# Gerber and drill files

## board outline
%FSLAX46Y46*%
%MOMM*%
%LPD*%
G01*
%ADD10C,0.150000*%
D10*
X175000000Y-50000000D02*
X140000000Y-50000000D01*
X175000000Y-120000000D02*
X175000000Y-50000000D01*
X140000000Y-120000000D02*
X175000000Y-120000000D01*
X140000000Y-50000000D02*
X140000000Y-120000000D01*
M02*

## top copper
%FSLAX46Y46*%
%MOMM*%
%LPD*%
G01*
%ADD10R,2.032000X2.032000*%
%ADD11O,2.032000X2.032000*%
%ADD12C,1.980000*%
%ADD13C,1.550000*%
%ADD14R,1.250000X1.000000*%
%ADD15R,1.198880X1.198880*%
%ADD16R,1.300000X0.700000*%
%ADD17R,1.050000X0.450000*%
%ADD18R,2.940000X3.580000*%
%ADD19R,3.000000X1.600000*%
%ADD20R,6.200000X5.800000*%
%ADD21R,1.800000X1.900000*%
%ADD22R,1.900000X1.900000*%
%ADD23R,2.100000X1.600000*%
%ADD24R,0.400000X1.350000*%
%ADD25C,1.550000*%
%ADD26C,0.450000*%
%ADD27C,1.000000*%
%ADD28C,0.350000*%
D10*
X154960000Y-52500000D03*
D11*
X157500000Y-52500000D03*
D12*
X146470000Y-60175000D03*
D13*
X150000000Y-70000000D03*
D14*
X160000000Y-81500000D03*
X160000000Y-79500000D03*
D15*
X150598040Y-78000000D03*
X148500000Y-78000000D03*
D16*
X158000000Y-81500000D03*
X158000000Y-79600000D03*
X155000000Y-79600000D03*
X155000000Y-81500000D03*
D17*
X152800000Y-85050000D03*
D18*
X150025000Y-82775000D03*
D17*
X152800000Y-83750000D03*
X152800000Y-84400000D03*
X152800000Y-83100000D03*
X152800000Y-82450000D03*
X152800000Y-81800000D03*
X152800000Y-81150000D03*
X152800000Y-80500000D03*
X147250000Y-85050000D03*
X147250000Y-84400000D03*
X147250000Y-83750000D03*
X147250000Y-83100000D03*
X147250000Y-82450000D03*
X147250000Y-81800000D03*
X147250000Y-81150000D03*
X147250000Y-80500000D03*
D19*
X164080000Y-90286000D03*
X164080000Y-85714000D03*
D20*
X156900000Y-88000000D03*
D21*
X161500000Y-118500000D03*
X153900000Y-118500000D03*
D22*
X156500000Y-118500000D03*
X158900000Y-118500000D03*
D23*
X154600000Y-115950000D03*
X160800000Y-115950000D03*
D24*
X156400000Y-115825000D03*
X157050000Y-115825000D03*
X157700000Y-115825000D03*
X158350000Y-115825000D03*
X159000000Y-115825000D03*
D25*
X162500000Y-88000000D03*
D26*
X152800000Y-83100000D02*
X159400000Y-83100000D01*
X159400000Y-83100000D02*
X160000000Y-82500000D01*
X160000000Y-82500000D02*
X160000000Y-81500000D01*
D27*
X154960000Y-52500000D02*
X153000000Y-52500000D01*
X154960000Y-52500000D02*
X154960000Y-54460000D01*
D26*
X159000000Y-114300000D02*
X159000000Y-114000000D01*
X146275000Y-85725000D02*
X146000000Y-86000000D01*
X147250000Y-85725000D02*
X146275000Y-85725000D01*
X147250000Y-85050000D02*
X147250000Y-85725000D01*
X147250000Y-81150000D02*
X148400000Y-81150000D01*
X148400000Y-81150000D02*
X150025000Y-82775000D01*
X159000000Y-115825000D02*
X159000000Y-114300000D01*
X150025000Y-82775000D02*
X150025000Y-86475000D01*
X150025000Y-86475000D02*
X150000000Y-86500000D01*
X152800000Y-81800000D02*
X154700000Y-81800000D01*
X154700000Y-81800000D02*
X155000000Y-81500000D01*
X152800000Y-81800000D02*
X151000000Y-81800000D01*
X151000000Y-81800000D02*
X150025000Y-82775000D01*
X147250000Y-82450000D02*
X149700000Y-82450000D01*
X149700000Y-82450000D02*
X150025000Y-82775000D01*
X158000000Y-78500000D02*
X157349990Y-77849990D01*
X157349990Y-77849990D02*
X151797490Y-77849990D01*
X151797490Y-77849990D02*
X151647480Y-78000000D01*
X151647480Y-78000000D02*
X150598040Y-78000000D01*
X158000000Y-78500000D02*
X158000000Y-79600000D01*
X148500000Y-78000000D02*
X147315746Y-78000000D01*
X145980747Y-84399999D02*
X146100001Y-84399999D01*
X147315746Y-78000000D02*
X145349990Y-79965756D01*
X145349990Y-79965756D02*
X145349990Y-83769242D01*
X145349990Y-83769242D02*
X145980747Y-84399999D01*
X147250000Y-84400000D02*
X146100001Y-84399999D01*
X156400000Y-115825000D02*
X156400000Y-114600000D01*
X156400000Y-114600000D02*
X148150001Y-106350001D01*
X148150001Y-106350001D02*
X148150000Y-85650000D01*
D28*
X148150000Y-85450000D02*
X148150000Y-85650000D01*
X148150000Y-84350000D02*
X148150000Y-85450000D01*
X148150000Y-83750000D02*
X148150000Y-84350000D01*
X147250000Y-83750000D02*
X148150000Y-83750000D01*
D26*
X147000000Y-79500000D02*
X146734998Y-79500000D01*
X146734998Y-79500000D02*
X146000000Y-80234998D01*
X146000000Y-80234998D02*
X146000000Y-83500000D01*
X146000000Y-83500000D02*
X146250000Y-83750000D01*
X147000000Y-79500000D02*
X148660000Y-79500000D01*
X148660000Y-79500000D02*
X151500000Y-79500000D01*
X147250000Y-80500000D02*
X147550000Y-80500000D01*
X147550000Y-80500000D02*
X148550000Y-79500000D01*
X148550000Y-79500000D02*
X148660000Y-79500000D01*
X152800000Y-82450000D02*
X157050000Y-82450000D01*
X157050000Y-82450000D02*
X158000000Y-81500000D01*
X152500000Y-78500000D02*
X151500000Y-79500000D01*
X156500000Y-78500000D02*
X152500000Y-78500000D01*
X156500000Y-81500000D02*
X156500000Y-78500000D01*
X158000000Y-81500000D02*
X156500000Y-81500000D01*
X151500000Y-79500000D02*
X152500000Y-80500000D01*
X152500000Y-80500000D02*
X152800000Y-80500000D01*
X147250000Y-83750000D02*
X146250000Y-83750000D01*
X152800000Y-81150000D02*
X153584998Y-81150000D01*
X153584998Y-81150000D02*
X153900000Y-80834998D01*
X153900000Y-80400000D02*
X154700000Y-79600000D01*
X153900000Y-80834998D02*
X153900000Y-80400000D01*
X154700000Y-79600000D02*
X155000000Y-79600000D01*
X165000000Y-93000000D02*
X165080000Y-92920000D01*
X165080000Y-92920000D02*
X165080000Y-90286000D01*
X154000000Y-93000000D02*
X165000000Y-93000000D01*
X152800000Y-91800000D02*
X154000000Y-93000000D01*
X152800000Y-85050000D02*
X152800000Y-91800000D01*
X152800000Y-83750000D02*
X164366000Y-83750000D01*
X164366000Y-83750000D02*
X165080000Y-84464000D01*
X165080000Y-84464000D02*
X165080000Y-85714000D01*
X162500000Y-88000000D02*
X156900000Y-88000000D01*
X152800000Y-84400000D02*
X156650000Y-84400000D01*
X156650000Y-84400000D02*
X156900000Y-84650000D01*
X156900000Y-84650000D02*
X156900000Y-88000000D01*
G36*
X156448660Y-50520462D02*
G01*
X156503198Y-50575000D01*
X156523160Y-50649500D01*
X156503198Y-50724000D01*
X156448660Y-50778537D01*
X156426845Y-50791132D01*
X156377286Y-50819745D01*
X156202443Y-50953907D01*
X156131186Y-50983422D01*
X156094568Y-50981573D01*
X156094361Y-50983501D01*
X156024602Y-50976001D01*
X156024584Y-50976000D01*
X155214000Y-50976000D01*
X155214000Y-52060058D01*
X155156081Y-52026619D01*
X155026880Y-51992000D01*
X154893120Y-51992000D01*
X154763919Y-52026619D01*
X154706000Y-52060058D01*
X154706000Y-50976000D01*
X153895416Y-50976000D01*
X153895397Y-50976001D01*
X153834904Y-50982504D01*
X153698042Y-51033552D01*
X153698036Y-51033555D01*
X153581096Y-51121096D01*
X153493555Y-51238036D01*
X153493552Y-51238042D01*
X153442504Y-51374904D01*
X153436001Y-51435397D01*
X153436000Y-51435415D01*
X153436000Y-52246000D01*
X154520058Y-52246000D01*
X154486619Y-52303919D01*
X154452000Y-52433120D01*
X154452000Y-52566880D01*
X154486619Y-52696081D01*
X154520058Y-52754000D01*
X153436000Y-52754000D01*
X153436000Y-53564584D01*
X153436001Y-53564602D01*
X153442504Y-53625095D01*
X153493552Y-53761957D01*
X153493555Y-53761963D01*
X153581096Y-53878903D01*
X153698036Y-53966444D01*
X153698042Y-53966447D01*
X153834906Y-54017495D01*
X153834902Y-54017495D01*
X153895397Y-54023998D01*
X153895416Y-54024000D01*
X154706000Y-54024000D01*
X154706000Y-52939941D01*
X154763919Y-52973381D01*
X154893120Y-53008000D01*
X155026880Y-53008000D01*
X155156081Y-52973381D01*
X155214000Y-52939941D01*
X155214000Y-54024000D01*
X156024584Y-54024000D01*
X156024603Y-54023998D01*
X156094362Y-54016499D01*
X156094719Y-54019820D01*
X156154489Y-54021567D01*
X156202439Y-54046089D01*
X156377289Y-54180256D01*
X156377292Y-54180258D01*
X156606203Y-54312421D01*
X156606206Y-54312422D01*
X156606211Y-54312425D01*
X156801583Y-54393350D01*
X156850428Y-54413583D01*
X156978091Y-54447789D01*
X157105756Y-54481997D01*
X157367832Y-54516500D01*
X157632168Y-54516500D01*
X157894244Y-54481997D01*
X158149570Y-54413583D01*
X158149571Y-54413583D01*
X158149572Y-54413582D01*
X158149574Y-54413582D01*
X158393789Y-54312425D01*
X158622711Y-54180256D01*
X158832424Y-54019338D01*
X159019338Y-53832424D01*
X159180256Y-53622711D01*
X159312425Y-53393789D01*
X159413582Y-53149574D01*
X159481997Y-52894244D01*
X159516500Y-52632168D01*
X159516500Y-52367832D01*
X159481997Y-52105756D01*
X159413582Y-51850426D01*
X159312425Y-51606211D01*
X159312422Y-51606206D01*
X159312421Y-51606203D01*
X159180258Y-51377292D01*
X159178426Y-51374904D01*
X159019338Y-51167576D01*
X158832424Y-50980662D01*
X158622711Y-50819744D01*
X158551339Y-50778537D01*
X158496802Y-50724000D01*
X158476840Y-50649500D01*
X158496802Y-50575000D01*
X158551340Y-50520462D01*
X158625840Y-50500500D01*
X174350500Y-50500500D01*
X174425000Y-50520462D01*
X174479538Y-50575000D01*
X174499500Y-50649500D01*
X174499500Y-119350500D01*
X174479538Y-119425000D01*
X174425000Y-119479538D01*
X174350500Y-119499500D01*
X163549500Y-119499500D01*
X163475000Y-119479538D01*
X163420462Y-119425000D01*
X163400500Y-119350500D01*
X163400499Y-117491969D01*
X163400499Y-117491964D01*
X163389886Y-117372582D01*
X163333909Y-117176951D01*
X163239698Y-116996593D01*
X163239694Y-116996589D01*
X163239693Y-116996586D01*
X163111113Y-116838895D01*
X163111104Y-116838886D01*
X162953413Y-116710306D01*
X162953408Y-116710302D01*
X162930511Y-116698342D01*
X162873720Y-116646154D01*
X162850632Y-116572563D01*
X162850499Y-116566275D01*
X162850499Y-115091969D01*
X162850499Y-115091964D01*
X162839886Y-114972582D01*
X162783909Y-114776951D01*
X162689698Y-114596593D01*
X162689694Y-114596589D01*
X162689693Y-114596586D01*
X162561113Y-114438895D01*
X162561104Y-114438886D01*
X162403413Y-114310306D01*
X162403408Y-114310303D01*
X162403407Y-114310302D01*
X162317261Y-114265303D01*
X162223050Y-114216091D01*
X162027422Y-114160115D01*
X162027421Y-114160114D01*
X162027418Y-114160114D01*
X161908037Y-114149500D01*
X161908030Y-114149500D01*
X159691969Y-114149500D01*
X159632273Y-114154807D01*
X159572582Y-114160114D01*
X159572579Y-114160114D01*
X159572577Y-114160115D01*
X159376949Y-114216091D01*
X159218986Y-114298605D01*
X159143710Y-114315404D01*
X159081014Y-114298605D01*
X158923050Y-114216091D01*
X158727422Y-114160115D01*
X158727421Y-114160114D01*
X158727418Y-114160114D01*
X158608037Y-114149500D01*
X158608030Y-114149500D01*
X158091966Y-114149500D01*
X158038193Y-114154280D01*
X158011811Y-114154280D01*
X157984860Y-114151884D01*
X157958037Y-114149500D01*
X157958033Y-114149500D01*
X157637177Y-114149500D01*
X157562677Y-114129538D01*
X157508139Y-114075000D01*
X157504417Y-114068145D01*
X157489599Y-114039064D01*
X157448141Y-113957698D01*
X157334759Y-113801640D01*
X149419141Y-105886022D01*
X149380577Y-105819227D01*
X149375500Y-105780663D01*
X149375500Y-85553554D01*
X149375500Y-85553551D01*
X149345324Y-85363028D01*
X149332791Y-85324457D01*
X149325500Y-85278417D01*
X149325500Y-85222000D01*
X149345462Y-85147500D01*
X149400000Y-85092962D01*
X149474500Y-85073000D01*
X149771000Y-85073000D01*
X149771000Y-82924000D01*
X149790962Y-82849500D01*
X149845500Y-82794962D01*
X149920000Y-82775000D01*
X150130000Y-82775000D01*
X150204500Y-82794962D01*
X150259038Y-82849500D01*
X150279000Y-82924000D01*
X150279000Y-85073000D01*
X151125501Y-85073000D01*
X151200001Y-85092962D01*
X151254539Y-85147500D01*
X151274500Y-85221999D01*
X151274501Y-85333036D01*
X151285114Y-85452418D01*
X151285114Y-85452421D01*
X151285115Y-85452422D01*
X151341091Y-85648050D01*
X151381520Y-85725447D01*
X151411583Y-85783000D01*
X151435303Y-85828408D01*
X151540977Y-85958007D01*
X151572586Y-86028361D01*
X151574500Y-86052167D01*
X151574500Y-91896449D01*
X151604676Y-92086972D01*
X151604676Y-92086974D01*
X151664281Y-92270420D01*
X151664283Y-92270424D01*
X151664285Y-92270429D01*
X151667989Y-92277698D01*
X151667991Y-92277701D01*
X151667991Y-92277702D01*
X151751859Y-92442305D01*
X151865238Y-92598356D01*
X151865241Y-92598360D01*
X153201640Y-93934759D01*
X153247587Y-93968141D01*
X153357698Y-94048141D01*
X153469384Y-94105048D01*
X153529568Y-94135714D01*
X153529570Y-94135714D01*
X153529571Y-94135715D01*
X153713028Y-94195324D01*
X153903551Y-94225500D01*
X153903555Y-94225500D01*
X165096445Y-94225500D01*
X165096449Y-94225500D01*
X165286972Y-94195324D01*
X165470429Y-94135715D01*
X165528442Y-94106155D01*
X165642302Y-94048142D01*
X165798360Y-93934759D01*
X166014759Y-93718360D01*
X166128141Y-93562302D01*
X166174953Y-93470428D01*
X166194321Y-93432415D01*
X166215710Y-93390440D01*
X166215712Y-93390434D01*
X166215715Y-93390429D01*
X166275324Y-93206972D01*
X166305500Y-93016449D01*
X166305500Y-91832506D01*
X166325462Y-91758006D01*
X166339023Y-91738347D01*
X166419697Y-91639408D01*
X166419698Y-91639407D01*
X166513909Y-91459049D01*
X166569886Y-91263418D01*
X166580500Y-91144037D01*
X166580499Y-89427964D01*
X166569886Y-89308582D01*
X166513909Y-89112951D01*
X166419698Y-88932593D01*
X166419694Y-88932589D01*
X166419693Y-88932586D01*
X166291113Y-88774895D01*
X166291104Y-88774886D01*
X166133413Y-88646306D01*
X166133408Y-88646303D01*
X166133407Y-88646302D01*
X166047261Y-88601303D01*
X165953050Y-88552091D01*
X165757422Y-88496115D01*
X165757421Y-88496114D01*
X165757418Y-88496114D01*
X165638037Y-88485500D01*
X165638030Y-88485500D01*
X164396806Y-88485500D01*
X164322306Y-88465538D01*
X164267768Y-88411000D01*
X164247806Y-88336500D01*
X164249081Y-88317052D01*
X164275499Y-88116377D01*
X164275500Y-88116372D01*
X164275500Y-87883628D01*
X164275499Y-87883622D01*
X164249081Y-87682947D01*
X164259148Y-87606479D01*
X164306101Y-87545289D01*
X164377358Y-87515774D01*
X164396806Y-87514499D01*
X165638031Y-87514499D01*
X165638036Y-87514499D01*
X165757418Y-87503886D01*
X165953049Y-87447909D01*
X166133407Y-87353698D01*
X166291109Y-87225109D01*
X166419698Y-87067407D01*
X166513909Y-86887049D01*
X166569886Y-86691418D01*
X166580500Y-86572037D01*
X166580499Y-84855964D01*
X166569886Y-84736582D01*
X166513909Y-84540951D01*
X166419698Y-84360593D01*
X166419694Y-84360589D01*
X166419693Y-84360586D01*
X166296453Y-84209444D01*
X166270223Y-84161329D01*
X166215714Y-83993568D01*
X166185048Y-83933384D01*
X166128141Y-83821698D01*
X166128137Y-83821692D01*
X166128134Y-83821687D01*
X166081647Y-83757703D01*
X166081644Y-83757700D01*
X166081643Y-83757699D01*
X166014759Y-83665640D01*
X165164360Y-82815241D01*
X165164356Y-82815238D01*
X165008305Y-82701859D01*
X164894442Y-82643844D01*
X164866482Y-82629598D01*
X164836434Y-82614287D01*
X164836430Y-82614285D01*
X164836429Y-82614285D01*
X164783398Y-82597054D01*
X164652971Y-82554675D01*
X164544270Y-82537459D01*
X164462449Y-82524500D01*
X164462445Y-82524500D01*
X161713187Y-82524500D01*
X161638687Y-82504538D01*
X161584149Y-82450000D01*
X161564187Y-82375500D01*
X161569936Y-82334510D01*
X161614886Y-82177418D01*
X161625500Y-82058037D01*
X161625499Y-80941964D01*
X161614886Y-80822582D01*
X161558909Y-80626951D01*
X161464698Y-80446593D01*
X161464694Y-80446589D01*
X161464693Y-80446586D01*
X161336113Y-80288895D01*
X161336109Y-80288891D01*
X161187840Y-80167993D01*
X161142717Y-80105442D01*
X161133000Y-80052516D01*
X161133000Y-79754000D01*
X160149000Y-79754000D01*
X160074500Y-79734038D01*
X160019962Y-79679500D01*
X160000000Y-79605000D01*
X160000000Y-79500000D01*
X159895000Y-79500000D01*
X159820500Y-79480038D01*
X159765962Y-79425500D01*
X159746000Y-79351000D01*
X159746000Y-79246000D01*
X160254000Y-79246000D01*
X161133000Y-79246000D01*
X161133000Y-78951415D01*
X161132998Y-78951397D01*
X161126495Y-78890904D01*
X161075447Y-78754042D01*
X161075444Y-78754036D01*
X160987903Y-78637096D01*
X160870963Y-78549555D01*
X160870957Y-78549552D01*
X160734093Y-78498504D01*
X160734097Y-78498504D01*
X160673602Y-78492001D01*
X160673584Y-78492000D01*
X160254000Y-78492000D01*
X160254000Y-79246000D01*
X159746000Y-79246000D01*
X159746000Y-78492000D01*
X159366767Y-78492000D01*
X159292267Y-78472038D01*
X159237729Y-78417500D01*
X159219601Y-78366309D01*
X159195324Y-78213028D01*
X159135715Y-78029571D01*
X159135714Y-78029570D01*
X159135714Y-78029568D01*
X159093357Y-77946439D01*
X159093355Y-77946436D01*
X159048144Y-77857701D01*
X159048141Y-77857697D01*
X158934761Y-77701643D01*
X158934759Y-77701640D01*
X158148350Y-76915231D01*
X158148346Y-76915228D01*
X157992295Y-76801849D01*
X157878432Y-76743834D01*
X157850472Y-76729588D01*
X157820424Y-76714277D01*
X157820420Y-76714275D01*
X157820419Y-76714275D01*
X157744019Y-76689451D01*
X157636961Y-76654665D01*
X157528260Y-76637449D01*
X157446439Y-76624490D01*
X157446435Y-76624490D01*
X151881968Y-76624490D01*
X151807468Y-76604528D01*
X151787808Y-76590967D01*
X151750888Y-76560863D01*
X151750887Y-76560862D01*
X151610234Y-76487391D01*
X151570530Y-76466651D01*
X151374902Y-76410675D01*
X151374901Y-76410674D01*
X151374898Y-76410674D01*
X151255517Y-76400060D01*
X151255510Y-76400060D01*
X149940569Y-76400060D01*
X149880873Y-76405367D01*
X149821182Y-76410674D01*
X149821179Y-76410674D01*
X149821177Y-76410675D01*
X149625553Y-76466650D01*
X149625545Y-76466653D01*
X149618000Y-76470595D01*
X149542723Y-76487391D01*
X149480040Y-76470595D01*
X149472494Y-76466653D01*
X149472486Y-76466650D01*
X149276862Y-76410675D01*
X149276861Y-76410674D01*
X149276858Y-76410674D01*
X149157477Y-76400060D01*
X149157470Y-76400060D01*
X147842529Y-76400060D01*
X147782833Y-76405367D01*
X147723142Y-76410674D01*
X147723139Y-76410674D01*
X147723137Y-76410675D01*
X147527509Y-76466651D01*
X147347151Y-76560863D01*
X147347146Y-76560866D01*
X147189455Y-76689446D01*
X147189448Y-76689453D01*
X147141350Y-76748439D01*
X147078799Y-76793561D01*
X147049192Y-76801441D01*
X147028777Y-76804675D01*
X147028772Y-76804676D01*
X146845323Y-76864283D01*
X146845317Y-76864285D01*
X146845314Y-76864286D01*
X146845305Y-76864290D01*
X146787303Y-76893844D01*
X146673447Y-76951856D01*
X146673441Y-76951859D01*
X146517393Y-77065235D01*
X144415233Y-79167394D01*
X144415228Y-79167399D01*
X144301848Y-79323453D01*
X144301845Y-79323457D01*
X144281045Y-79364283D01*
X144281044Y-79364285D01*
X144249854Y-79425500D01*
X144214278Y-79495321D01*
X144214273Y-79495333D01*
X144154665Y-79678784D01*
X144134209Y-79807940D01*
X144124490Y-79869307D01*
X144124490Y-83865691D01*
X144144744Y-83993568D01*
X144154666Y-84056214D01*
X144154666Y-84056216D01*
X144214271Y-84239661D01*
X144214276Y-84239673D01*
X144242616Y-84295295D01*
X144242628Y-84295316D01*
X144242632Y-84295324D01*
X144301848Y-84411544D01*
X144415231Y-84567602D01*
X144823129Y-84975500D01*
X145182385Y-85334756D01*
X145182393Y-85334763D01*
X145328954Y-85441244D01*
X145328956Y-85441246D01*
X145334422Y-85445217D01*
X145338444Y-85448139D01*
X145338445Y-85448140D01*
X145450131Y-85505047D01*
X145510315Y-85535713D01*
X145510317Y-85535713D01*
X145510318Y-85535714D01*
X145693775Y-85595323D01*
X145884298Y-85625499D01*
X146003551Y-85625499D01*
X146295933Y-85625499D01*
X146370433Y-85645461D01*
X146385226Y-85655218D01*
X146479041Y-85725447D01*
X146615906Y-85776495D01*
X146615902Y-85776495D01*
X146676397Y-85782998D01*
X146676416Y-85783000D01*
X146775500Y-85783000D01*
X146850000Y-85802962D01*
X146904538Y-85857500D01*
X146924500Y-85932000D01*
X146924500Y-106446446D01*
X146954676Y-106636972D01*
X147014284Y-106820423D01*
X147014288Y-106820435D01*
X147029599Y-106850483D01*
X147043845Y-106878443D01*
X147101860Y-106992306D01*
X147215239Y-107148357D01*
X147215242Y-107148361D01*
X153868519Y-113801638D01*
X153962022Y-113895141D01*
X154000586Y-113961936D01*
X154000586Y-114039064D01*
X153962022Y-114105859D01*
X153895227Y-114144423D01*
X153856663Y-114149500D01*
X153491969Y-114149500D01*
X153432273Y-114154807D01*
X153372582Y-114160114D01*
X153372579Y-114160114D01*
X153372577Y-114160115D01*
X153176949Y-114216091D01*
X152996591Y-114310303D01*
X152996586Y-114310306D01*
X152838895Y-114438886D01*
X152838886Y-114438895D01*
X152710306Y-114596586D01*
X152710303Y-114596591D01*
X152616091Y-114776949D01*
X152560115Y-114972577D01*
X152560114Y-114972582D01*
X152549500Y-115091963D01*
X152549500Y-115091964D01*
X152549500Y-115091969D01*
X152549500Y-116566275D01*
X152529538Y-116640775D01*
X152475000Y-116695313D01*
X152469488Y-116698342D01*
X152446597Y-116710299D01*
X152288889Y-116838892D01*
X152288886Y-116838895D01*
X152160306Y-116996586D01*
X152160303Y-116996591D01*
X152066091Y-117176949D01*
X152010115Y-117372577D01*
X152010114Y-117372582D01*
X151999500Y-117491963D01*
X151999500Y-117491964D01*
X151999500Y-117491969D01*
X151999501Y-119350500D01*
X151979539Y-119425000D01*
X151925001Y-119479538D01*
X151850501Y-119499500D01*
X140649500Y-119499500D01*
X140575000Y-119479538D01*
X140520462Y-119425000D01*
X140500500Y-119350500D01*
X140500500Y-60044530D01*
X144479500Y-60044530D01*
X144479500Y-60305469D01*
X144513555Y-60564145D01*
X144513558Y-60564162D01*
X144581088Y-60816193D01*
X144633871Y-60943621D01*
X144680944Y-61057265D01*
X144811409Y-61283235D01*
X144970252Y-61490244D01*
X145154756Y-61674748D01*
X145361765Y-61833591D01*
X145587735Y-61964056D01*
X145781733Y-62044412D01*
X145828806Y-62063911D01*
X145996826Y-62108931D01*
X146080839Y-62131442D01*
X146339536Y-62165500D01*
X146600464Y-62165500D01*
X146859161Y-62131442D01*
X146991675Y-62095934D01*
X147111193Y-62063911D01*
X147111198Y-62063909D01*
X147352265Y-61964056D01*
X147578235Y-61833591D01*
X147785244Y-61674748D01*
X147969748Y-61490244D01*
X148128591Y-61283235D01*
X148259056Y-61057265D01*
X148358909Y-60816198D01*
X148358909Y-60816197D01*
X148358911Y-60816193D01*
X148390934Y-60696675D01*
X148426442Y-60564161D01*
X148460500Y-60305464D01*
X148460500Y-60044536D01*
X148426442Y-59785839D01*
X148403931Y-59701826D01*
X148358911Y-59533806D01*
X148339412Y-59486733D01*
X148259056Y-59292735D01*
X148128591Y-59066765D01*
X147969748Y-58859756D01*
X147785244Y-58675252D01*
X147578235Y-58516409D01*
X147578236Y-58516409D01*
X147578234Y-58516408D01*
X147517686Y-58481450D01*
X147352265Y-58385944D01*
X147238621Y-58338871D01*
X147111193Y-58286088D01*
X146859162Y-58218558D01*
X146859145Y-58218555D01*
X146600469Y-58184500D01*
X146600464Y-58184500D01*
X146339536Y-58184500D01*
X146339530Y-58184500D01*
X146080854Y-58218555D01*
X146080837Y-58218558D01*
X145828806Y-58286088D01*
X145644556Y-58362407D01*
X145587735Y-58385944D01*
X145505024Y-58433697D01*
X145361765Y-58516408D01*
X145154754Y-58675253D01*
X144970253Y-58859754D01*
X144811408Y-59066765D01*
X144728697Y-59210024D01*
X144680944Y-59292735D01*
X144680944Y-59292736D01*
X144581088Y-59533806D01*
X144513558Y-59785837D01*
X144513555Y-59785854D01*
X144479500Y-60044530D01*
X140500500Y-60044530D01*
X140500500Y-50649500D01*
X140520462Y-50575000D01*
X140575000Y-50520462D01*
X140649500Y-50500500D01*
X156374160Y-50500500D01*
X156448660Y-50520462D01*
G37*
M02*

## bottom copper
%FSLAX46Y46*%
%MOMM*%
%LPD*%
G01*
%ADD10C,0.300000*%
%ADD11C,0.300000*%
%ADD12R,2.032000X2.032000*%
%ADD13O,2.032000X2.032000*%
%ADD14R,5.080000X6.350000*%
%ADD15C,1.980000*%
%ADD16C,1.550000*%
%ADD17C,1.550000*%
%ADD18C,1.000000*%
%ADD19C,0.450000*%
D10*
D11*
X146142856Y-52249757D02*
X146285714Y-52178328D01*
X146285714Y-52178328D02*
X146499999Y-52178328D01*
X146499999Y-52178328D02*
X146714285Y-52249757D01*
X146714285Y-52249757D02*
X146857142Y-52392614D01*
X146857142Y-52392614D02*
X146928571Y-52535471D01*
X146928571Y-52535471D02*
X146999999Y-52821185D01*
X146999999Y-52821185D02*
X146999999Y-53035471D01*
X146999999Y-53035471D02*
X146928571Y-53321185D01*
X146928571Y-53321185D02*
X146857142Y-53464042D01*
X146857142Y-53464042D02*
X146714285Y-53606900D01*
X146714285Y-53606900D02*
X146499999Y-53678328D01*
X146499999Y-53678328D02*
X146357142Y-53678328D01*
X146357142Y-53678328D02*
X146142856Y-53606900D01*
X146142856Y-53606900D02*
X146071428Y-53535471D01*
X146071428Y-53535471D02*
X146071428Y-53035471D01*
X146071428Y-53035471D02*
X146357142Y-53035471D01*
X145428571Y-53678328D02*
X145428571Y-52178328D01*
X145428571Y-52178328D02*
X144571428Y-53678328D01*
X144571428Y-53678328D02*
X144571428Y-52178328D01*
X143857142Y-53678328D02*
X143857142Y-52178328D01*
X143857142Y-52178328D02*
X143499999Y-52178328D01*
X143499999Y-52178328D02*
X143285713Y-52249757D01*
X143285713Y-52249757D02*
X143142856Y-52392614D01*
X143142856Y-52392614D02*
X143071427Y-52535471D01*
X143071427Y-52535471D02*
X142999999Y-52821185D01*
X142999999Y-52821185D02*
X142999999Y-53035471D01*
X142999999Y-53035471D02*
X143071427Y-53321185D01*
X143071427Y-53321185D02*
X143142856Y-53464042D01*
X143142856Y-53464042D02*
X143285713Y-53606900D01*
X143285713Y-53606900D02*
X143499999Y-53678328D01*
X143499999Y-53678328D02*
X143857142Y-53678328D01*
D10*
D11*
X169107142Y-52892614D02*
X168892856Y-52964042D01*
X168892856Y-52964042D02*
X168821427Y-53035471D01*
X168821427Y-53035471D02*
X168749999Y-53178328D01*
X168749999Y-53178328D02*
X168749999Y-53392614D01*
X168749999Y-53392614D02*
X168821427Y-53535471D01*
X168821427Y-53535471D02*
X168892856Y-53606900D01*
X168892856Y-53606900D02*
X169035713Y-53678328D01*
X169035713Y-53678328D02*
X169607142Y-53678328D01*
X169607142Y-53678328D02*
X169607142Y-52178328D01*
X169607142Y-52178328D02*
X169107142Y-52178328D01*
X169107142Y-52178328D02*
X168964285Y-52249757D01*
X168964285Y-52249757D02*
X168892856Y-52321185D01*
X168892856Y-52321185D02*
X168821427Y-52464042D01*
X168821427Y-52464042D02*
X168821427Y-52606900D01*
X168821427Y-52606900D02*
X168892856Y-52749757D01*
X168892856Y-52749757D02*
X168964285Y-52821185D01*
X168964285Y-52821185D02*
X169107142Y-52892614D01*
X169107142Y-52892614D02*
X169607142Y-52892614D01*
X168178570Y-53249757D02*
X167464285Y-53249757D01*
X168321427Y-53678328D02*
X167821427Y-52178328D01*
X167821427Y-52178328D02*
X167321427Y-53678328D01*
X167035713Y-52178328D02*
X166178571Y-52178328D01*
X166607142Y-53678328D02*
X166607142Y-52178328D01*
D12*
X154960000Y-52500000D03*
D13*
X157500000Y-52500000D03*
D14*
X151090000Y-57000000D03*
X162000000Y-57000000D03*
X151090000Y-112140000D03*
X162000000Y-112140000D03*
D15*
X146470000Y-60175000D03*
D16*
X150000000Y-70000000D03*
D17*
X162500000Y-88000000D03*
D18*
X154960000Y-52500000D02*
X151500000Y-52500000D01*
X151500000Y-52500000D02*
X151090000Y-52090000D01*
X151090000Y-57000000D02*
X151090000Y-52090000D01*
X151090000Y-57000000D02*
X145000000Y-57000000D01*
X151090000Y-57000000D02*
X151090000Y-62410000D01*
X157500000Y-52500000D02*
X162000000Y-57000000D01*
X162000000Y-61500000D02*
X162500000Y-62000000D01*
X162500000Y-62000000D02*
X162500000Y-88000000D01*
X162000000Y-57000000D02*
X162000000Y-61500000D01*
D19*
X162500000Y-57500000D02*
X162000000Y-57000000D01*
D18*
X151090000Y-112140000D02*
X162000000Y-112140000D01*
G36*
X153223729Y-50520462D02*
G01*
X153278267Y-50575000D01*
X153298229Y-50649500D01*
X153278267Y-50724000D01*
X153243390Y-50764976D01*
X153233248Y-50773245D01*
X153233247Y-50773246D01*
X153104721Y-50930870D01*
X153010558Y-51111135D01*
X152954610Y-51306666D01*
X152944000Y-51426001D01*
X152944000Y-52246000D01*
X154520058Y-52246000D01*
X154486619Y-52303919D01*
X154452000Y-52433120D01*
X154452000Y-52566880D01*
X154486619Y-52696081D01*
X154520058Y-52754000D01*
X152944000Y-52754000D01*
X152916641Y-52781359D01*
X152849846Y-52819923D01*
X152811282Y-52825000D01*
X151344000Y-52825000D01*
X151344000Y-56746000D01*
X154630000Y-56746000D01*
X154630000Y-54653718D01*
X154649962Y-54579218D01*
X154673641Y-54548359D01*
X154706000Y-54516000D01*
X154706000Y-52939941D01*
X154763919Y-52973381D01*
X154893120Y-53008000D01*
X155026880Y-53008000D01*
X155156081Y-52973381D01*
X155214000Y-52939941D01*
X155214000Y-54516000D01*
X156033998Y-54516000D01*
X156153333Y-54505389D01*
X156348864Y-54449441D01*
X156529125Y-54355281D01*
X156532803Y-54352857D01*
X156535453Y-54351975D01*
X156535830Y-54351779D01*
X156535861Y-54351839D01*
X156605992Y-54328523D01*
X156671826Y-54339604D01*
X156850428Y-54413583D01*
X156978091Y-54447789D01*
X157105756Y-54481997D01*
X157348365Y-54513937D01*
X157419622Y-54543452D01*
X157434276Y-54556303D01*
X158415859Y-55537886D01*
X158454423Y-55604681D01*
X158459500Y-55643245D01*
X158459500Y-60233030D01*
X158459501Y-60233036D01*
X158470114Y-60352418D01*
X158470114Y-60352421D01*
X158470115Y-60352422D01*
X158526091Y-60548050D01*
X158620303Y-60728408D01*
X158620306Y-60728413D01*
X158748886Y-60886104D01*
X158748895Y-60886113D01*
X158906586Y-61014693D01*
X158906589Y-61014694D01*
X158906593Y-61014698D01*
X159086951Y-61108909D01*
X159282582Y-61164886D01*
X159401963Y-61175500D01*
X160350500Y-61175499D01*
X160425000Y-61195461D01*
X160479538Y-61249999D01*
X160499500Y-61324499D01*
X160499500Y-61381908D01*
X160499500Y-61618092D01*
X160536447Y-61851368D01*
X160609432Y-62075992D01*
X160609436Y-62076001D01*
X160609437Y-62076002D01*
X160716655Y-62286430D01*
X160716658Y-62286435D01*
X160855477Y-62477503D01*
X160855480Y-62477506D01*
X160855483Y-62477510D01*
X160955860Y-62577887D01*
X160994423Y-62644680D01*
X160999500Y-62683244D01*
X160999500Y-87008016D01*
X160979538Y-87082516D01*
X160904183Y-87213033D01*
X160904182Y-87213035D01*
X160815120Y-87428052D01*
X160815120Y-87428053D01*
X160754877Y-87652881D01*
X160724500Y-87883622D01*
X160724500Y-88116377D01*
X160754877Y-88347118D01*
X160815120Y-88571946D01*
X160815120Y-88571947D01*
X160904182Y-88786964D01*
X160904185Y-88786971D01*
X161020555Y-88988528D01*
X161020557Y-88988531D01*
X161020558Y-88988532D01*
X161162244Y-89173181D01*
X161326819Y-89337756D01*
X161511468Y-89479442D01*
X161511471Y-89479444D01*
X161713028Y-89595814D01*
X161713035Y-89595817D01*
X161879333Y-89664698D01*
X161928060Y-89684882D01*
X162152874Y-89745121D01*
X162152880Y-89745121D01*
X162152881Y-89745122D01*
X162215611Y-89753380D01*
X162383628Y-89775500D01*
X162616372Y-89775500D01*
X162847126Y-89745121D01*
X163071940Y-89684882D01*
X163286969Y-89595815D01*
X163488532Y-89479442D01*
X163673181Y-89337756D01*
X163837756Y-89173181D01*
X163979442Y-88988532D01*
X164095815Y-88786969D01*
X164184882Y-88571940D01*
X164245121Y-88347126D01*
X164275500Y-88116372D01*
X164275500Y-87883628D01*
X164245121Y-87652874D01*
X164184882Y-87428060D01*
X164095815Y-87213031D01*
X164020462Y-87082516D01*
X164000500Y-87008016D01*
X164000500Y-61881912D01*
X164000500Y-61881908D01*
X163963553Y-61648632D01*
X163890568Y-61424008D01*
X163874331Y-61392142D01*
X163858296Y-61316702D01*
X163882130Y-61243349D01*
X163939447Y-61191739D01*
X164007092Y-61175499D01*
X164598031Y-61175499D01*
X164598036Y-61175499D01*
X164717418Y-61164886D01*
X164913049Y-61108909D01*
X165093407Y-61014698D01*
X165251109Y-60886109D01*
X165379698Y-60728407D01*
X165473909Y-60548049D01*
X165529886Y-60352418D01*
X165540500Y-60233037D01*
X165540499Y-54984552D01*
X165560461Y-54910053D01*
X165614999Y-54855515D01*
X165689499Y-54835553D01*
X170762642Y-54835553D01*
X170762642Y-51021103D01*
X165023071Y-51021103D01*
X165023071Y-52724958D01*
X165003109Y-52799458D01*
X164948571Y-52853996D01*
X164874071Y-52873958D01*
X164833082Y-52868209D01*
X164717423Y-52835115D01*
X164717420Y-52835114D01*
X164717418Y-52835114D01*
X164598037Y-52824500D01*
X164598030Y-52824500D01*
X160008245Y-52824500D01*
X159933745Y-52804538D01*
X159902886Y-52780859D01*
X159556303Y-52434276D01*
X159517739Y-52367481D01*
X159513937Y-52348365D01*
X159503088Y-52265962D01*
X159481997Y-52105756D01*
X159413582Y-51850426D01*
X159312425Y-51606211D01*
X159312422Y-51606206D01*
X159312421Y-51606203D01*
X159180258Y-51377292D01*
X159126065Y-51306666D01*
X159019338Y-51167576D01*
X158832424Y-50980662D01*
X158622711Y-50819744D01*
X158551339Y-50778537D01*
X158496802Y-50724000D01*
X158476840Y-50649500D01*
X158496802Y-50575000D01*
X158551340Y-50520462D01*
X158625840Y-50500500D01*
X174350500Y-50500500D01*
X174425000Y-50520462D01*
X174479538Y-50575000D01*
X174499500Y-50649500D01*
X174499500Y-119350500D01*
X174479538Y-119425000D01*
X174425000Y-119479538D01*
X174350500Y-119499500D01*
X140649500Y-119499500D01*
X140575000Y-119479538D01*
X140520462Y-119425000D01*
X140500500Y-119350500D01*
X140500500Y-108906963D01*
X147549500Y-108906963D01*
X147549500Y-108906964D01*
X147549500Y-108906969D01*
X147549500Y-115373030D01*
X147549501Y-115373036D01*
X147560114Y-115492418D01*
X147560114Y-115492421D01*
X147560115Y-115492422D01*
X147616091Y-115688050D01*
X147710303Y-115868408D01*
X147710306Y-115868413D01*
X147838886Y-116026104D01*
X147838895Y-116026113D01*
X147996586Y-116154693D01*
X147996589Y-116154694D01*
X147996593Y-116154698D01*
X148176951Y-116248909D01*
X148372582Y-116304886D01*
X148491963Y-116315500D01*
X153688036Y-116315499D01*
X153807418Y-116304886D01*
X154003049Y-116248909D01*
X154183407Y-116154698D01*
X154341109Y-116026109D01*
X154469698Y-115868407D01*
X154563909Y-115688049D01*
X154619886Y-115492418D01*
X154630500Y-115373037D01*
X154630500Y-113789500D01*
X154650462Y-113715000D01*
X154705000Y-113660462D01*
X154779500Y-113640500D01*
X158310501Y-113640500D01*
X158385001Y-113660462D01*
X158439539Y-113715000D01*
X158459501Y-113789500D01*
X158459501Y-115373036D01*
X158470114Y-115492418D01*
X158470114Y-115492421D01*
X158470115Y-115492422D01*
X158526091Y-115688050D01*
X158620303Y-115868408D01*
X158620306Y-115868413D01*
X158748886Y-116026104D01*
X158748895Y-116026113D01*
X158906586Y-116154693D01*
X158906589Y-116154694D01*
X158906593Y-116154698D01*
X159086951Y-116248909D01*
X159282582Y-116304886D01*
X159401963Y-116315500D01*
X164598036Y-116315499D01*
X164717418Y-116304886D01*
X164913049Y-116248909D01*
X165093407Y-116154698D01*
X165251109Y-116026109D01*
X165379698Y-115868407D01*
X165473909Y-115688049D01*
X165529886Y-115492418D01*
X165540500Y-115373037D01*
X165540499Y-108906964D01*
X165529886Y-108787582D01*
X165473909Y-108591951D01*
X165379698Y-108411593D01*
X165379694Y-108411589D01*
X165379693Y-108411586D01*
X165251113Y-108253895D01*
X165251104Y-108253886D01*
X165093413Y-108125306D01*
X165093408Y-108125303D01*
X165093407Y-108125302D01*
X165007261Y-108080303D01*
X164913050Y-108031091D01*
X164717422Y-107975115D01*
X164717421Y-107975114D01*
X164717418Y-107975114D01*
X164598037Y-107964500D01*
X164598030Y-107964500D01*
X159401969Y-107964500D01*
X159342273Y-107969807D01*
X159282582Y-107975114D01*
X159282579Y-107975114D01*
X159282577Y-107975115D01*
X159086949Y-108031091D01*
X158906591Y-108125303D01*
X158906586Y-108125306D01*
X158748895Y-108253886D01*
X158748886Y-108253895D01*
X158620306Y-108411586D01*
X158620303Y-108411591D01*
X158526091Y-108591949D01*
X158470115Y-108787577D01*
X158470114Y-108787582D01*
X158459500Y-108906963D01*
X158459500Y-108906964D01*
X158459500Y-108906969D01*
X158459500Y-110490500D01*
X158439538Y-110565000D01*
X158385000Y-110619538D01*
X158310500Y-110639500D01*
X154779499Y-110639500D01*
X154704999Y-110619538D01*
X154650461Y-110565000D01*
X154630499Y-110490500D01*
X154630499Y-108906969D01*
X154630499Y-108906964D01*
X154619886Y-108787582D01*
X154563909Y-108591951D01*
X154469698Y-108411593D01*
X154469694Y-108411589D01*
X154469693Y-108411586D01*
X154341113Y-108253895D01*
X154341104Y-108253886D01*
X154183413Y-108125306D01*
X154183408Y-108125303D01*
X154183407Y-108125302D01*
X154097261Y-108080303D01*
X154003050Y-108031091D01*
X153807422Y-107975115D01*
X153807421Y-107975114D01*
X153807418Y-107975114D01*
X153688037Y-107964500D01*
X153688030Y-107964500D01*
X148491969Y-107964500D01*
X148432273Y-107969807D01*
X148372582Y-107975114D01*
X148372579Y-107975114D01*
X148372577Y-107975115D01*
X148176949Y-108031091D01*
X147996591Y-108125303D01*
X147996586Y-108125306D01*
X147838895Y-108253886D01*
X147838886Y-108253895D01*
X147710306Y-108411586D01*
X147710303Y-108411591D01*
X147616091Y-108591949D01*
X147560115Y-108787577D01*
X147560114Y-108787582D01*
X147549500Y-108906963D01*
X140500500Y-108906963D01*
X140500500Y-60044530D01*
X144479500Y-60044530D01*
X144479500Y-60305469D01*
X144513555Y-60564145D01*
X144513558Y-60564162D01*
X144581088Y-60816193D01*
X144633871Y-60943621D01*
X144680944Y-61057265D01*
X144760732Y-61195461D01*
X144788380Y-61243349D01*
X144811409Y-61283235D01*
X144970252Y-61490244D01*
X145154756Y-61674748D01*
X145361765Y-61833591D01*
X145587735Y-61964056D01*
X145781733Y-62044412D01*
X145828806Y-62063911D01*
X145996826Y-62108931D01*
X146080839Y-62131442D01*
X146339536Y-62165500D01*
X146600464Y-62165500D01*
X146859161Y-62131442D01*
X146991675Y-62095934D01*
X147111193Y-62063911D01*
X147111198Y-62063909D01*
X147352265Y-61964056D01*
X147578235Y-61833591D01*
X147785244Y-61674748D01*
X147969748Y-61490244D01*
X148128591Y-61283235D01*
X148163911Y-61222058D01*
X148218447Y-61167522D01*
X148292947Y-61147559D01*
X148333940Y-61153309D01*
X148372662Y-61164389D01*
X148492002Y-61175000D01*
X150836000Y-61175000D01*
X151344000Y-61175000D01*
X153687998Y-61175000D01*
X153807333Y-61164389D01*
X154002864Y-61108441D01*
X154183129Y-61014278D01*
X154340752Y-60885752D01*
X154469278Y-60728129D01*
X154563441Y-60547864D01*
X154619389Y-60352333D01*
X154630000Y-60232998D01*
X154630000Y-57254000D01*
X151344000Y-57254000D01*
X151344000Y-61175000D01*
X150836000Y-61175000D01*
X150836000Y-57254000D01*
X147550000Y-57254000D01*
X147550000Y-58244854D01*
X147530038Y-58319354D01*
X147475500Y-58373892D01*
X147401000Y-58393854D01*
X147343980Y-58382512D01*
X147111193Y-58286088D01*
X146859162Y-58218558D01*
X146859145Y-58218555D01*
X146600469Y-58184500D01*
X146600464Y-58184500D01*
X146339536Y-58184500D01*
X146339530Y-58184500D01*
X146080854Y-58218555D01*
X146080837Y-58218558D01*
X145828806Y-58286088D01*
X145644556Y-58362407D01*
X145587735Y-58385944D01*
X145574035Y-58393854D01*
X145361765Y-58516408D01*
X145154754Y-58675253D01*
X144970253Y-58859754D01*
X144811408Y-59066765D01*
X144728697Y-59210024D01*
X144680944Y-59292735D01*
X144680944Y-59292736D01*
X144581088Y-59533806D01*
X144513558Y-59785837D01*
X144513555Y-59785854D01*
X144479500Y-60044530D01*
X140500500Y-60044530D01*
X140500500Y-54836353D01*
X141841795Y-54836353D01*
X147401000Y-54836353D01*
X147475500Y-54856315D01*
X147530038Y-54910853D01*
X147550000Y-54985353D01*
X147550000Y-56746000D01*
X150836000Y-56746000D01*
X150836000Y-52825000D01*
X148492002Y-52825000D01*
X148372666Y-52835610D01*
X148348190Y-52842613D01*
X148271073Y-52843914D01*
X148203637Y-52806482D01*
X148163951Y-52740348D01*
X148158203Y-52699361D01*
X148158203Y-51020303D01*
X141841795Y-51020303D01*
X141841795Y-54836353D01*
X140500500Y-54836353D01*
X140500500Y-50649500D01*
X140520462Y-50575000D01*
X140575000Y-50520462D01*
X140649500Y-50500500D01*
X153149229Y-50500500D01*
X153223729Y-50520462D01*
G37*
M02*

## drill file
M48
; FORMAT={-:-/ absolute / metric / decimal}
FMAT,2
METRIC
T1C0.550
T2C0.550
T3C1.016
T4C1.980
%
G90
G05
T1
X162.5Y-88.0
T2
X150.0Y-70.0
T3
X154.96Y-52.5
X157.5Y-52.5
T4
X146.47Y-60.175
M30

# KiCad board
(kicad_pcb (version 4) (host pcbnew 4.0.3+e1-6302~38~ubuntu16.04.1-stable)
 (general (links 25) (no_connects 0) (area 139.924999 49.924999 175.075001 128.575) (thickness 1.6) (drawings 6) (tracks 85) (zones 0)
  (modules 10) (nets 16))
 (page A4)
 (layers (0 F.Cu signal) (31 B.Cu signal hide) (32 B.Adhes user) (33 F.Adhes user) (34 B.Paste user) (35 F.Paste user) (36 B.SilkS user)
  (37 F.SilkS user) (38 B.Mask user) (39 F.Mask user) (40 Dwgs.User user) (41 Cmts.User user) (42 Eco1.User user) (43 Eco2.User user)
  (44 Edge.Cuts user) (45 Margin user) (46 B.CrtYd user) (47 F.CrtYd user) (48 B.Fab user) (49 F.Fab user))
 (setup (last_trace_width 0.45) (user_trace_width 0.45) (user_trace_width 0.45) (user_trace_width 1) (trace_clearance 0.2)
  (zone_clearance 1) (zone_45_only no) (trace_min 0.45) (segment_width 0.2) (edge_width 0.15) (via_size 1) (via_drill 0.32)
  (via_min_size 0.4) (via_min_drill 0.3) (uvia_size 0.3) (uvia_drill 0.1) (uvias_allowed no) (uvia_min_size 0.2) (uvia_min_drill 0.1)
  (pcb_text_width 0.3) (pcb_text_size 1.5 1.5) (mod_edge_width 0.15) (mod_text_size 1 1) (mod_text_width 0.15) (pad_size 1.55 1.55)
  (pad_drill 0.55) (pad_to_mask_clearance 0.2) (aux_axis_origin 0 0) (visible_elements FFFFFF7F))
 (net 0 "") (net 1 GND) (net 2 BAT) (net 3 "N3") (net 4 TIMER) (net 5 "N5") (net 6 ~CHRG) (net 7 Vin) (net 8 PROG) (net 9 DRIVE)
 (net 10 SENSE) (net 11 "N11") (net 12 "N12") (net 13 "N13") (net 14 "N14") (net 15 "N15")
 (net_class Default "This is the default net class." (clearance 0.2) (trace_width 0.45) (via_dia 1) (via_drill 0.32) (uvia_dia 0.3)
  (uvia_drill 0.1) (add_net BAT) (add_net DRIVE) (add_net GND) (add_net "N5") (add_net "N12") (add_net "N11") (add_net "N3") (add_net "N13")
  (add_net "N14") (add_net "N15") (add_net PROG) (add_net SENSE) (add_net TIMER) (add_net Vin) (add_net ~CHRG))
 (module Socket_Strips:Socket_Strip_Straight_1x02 (layer B.Cu) (at 154.96 52.5)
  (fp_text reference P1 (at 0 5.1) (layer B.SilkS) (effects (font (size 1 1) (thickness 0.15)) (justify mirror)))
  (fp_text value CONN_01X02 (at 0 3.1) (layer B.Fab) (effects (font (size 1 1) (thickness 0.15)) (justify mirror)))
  (pad 1 thru_hole rect (at 0 0) (size 2.032 2.032) (drill 1.016) (layers *.Cu *.Mask B.SilkS) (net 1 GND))
  (pad 2 thru_hole oval (at 2.54 0) (size 2.032 2.032) (drill 1.016) (layers *.Cu *.Mask B.SilkS) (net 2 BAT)))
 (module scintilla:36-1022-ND (layer B.Cu) (at 156.545 84.57 270)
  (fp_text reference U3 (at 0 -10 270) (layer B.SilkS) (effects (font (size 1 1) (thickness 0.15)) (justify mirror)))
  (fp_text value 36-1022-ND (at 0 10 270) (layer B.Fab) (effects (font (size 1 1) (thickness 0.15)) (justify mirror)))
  (pad 2 smd rect (at -27.57 5.455 270) (size 6.35 5.08) (layers B.Cu B.Paste B.Mask) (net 1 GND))
  (pad 1 smd rect (at -27.57 -5.455 270) (size 6.35 5.08) (layers B.Cu B.Paste B.Mask) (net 2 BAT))
  (pad 3 smd rect (at 27.57 5.455 270) (size 6.35 5.08) (layers B.Cu B.Paste B.Mask) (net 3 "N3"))
  (pad 4 smd rect (at 27.57 -5.455 270) (size 6.35 5.08) (layers B.Cu B.Paste B.Mask) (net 3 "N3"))
  (pad 5 thru_hole circle (at -24.395 10.075 270) (size 1.98 1.98) (drill 1.98) (layers *.Cu *.Mask)))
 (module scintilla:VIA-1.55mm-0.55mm (layer F.Cu) (at 150 70)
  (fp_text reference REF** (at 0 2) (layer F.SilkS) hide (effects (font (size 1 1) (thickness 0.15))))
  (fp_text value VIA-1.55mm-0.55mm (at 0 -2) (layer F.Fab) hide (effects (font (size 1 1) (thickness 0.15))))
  (pad 1 thru_hole circle (at 0 0) (size 1.55 1.55) (drill 0.55) (layers *.Cu) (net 1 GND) (zone_connect 2)))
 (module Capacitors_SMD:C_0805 (layer F.Cu) (at 160 80.5 90)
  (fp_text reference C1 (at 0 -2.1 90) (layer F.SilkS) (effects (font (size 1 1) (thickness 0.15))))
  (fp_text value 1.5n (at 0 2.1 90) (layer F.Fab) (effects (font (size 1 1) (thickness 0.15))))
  (pad 1 smd rect (at -1 0 90) (size 1 1.25) (layers F.Cu F.Paste F.Mask) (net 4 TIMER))
  (pad 2 smd rect (at 1 0 90) (size 1 1.25) (layers F.Cu F.Paste F.Mask) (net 1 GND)))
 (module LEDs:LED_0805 (layer F.Cu) (at 149.54902 78)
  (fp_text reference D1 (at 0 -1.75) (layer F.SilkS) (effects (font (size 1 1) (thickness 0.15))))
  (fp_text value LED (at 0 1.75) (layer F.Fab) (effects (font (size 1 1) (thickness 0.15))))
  (pad 2 smd rect (at 1.04902 0 180) (size 1.19888 1.19888) (layers F.Cu F.Paste F.Mask) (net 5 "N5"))
  (pad 1 smd rect (at -1.04902 0 180) (size 1.19888 1.19888) (layers F.Cu F.Paste F.Mask) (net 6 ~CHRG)))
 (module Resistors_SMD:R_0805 (layer F.Cu) (at 158 80.55 90)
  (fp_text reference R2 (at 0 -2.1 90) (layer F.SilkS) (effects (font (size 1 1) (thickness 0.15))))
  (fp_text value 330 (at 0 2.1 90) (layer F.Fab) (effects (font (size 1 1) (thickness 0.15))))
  (pad 1 smd rect (at -0.95 0 90) (size 0.7 1.3) (layers F.Cu F.Paste F.Mask) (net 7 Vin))
  (pad 2 smd rect (at 0.95 0 90) (size 0.7 1.3) (layers F.Cu F.Paste F.Mask) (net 5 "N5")))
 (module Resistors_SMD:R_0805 (layer F.Cu) (at 155 80.55 270)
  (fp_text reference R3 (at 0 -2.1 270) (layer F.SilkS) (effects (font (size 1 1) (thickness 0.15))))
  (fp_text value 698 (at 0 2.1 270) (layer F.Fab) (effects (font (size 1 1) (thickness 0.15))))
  (pad 1 smd rect (at -0.95 0 270) (size 0.7 1.3) (layers F.Cu F.Paste F.Mask) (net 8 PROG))
  (pad 2 smd rect (at 0.95 0 270) (size 0.7 1.3) (layers F.Cu F.Paste F.Mask) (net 1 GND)))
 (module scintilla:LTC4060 (layer F.Cu) (at 150.025 82.775 90)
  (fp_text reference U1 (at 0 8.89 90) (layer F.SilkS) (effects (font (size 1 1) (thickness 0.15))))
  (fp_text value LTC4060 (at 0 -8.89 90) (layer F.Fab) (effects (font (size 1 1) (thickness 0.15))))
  (pad 1 smd rect (at -2.275 2.775 90) (size 0.45 1.05) (layers F.Cu F.Paste F.Mask) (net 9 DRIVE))
  (pad 17 smd rect (at 0 0 90) (size 3.58 2.94) (layers F.Cu F.Paste F.Mask) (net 1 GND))
  (pad 3 smd rect (at -0.975 2.775 90) (size 0.45 1.05) (layers F.Cu F.Paste F.Mask) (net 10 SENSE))
  (pad 2 smd rect (at -1.625 2.775 90) (size 0.45 1.05) (layers F.Cu F.Paste F.Mask) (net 2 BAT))
  (pad 4 smd rect (at -0.325 2.775 90) (size 0.45 1.05) (layers F.Cu F.Paste F.Mask) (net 4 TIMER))
  (pad 5 smd rect (at 0.325 2.775 90) (size 0.45 1.05) (layers F.Cu F.Paste F.Mask) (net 7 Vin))
  (pad 6 smd rect (at 0.975 2.775 90) (size 0.45 1.05) (layers F.Cu F.Paste F.Mask) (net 1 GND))
  (pad 7 smd rect (at 1.625 2.775 90) (size 0.45 1.05) (layers F.Cu F.Paste F.Mask) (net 8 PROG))
  (pad 8 smd rect (at 2.275 2.775 90) (size 0.45 1.05) (layers F.Cu F.Paste F.Mask) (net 7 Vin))
  (pad 16 smd rect (at -2.275 -2.775 90) (size 0.45 1.05) (layers F.Cu F.Paste F.Mask) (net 1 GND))
  (pad 15 smd rect (at -1.625 -2.775 90) (size 0.45 1.05) (layers F.Cu F.Paste F.Mask) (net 6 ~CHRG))
  (pad 14 smd rect (at -0.975 -2.775 90) (size 0.45 1.05) (layers F.Cu F.Paste F.Mask) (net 7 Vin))
  (pad 13 smd rect (at -0.325 -2.775 90) (size 0.45 1.05) (layers F.Cu F.Paste F.Mask) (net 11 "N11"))
  (pad 12 smd rect (at 0.325 -2.775 90) (size 0.45 1.05) (layers F.Cu F.Paste F.Mask) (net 1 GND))
  (pad 11 smd rect (at 0.975 -2.775 90) (size 0.45 1.05) (layers F.Cu F.Paste F.Mask) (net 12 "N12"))
  (pad 10 smd rect (at 1.625 -2.775 90) (size 0.45 1.05) (layers F.Cu F.Paste F.Mask) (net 1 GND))
  (pad 9 smd rect (at 2.275 -2.775 90) (size 0.45 1.05) (layers F.Cu F.Paste F.Mask) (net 7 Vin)))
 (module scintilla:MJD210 (layer F.Cu) (at 160 88)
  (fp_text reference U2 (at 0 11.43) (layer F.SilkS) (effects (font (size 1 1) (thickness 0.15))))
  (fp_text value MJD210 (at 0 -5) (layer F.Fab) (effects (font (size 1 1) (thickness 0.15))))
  (pad 1 smd rect (at 4.08 2.286) (size 3 1.6) (layers F.Cu F.Paste F.Mask) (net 9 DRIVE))
  (pad 3 smd rect (at 4.08 -2.286) (size 3 1.6) (layers F.Cu F.Paste F.Mask) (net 10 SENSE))
  (pad 4 smd rect (at -3.1 0) (size 6.2 5.8) (layers F.Cu F.Paste F.Mask) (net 2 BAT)))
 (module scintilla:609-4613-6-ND (layer F.Cu) (at 157.7 118.5)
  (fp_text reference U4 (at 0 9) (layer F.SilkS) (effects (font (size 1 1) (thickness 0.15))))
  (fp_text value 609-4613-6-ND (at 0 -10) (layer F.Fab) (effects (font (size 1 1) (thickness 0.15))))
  (pad "" smd rect (at 3.8 0) (size 1.8 1.9) (layers F.Cu F.Paste F.Mask))
  (pad "" smd rect (at -3.8 0) (size 1.8 1.9) (layers F.Cu F.Paste F.Mask))
  (pad "" smd rect (at -1.2 0) (size 1.9 1.9) (layers F.Cu F.Paste F.Mask))
  (pad "" smd rect (at 1.2 0) (size 1.9 1.9) (layers F.Cu F.Paste F.Mask))
  (pad "" smd rect (at -3.1 -2.55) (size 2.1 1.6) (layers F.Cu F.Paste F.Mask))
  (pad "" smd rect (at 3.1 -2.55) (size 2.1 1.6) (layers F.Cu F.Paste F.Mask))
  (pad 1 smd rect (at -1.3 -2.675) (size 0.4 1.35) (layers F.Cu F.Paste F.Mask) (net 7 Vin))
  (pad 2 smd rect (at -0.65 -2.675) (size 0.4 1.35) (layers F.Cu F.Paste F.Mask) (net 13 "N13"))
  (pad 3 smd rect (at 0 -2.675) (size 0.4 1.35) (layers F.Cu F.Paste F.Mask) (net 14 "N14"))
  (pad 4 smd rect (at 0.65 -2.675) (size 0.4 1.35) (layers F.Cu F.Paste F.Mask) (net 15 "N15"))
  (pad 5 smd rect (at 1.3 -2.675) (size 0.4 1.35) (layers F.Cu F.Paste F.Mask) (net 1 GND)))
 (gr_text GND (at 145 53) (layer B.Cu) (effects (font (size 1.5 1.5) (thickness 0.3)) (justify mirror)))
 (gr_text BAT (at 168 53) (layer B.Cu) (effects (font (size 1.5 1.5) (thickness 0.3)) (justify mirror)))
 (gr_line (start 175 50) (end 140 50) (layer Edge.Cuts) (width 0.15))
 (gr_line (start 175 120) (end 175 50) (layer Edge.Cuts) (width 0.15))
 (gr_line (start 140 120) (end 175 120) (layer Edge.Cuts) (width 0.15))
 (gr_line (start 140 50) (end 140 120) (layer Edge.Cuts) (width 0.15))
 (segment (start 152.8 83.1) (end 159.4 83.1) (width 0.45) (layer F.Cu) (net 4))
 (segment (start 159.4 83.1) (end 160 82.5) (width 0.45) (layer F.Cu) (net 4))
 (segment (start 160 82.5) (end 160 81.5) (width 0.45) (layer F.Cu) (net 4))
 (segment (start 154.96 52.5) (end 153 52.5) (width 1) (layer F.Cu) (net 1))
 (segment (start 154.96 52.5) (end 154.96 54.46) (width 1) (layer F.Cu) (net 1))
 (segment (start 154.96 52.5) (end 151.5 52.5) (width 1) (layer B.Cu) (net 1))
 (segment (start 151.5 52.5) (end 151.09 52.09) (width 1) (layer B.Cu) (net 1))
 (segment (start 151.09 57) (end 151.09 52.09) (width 1) (layer B.Cu) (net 1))
 (segment (start 151.09 57) (end 145 57) (width 1) (layer B.Cu) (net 1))
 (segment (start 151.09 57) (end 151.09 62.41) (width 1) (layer B.Cu) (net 1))
 (segment (start 159 114.3) (end 159 114) (width 0.45) (layer F.Cu) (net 1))
 (segment (start 146.275 85.725) (end 146 86) (width 0.45) (layer F.Cu) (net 1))
 (segment (start 147.25 85.725) (end 146.275 85.725) (width 0.45) (layer F.Cu) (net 1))
 (segment (start 147.25 85.05) (end 147.25 85.725) (width 0.45) (layer F.Cu) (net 1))
 (segment (start 147.25 81.15) (end 148.4 81.15) (width 0.45) (layer F.Cu) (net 1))
 (segment (start 148.4 81.15) (end 150.025 82.775) (width 0.45) (layer F.Cu) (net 1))
 (segment (start 159 115.825) (end 159 114.3) (width 0.45) (layer F.Cu) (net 1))
 (segment (start 150.025 82.775) (end 150.025 86.475) (width 0.45) (layer F.Cu) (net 1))
 (segment (start 150.025 86.475) (end 150 86.5) (width 0.45) (layer F.Cu) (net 1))
 (segment (start 152.8 81.8) (end 154.7 81.8) (width 0.45) (layer F.Cu) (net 1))
 (segment (start 154.7 81.8) (end 155 81.5) (width 0.45) (layer F.Cu) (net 1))
 (segment (start 152.8 81.8) (end 151 81.8) (width 0.45) (layer F.Cu) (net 1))
 (segment (start 151 81.8) (end 150.025 82.775) (width 0.45) (layer F.Cu) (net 1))
 (segment (start 147.25 82.45) (end 149.7 82.45) (width 0.45) (layer F.Cu) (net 1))
 (segment (start 149.7 82.45) (end 150.025 82.775) (width 0.45) (layer F.Cu) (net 1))
 (segment (start 158 78.5) (end 157.34999 77.84999) (width 0.45) (layer F.Cu) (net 5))
 (segment (start 157.34999 77.84999) (end 151.79749 77.84999) (width 0.45) (layer F.Cu) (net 5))
 (segment (start 151.79749 77.84999) (end 151.64748 78) (width 0.45) (layer F.Cu) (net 5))
 (segment (start 151.64748 78) (end 150.59804 78) (width 0.45) (layer F.Cu) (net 5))
 (segment (start 158 78.5) (end 158 79.6) (width 0.45) (layer F.Cu) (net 5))
 (segment (start 148.5 78) (end 147.315746 78) (width 0.45) (layer F.Cu) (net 6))
 (segment (start 145.980747 84.399999) (end 146.100001 84.399999) (width 0.45) (layer F.Cu) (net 6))
 (segment (start 147.315746 78) (end 145.34999 79.965756) (width 0.45) (layer F.Cu) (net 6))
 (segment (start 145.34999 79.965756) (end 145.34999 83.769242) (width 0.45) (layer F.Cu) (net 6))
 (segment (start 145.34999 83.769242) (end 145.980747 84.399999) (width 0.45) (layer F.Cu) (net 6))
 (segment (start 147.25 84.4) (end 146.100001 84.399999) (width 0.45) (layer F.Cu) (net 6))
 (segment (start 156.4 115.825) (end 156.4 114.6) (width 0.45) (layer F.Cu) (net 7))
 (segment (start 156.4 114.6) (end 148.150001 106.350001) (width 0.45) (layer F.Cu) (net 7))
 (segment (start 148.150001 106.350001) (end 148.15 85.65) (width 0.45) (layer F.Cu) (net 7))
 (segment (start 148.15 85.45) (end 148.15 85.65) (width 0.35) (layer F.Cu) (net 7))
 (segment (start 148.15 84.35) (end 148.15 85.45) (width 0.35) (layer F.Cu) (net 7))
 (segment (start 148.15 83.75) (end 148.15 84.35) (width 0.35) (layer F.Cu) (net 7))
 (segment (start 147.25 83.75) (end 148.15 83.75) (width 0.35) (layer F.Cu) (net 7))
 (segment (start 147 79.5) (end 146.734998 79.5) (width 0.45) (layer F.Cu) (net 7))
 (segment (start 146.734998 79.5) (end 146 80.234998) (width 0.45) (layer F.Cu) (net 7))
 (segment (start 146 80.234998) (end 146 83.5) (width 0.45) (layer F.Cu) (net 7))
 (segment (start 146 83.5) (end 146.25 83.75) (width 0.45) (layer F.Cu) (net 7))
 (segment (start 147 79.5) (end 148.66 79.5) (width 0.45) (layer F.Cu) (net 7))
 (segment (start 148.66 79.5) (end 151.5 79.5) (width 0.45) (layer F.Cu) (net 7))
 (segment (start 147.25 80.5) (end 147.55 80.5) (width 0.45) (layer F.Cu) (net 7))
 (segment (start 147.55 80.5) (end 148.55 79.5) (width 0.45) (layer F.Cu) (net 7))
 (segment (start 148.55 79.5) (end 148.66 79.5) (width 0.45) (layer F.Cu) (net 7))
 (segment (start 152.8 82.45) (end 157.05 82.45) (width 0.45) (layer F.Cu) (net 7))
 (segment (start 157.05 82.45) (end 158 81.5) (width 0.45) (layer F.Cu) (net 7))
 (segment (start 152.5 78.5) (end 151.5 79.5) (width 0.45) (layer F.Cu) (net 7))
 (segment (start 156.5 78.5) (end 152.5 78.5) (width 0.45) (layer F.Cu) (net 7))
 (segment (start 156.5 81.5) (end 156.5 78.5) (width 0.45) (layer F.Cu) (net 7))
 (segment (start 158 81.5) (end 156.5 81.5) (width 0.45) (layer F.Cu) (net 7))
 (segment (start 151.5 79.5) (end 152.5 80.5) (width 0.45) (layer F.Cu) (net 7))
 (segment (start 152.5 80.5) (end 152.8 80.5) (width 0.45) (layer F.Cu) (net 7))
 (segment (start 147.25 83.75) (end 146.25 83.75) (width 0.45) (layer F.Cu) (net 7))
 (segment (start 152.8 81.15) (end 153.584998 81.15) (width 0.45) (layer F.Cu) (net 8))
 (segment (start 153.584998 81.15) (end 153.9 80.834998) (width 0.45) (layer F.Cu) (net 8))
 (segment (start 153.9 80.4) (end 154.7 79.6) (width 0.45) (layer F.Cu) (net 8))
 (segment (start 153.9 80.834998) (end 153.9 80.4) (width 0.45) (layer F.Cu) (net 8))
 (segment (start 154.7 79.6) (end 155 79.6) (width 0.45) (layer F.Cu) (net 8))
 (segment (start 165 93) (end 165.08 92.92) (width 0.45) (layer F.Cu) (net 9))
 (segment (start 165.08 92.92) (end 165.08 90.286) (width 0.45) (layer F.Cu) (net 9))
 (segment (start 154 93) (end 165 93) (width 0.45) (layer F.Cu) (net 9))
 (segment (start 152.8 91.8) (end 154 93) (width 0.45) (layer F.Cu) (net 9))
 (segment (start 152.8 85.05) (end 152.8 91.8) (width 0.45) (layer F.Cu) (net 9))
 (segment (start 152.8 83.75) (end 164.366 83.75) (width 0.45) (layer F.Cu) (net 10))
 (segment (start 164.366 83.75) (end 165.08 84.464) (width 0.45) (layer F.Cu) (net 10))
 (segment (start 165.08 84.464) (end 165.08 85.714) (width 0.45) (layer F.Cu) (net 10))
 (segment (start 157.5 52.5) (end 162 57) (width 1) (layer B.Cu) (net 2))
 (segment (start 162 61.5) (end 162.5 62) (width 1) (layer B.Cu) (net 2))
 (segment (start 162.5 62) (end 162.5 88) (width 1) (layer B.Cu) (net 2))
 (segment (start 162 57) (end 162 61.5) (width 1) (layer B.Cu) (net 2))
 (segment (start 162.5 88) (end 156.9 88) (width 0.45) (layer F.Cu) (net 2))
 (segment (start 152.8 84.4) (end 156.65 84.4) (width 0.45) (layer F.Cu) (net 2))
 (segment (start 156.65 84.4) (end 156.9 84.65) (width 0.45) (layer F.Cu) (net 2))
 (segment (start 156.9 84.65) (end 156.9 88) (width 0.45) (layer F.Cu) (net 2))
 (via (at 162.5 88) (size 1.55) (drill 0.55) (layers F.Cu B.Cu) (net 2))
 (segment (start 162.5 57.5) (end 162 57) (width 0.45) (layer B.Cu) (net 2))
 (segment (start 151.09 112.14) (end 162 112.14) (width 1) (layer B.Cu) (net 3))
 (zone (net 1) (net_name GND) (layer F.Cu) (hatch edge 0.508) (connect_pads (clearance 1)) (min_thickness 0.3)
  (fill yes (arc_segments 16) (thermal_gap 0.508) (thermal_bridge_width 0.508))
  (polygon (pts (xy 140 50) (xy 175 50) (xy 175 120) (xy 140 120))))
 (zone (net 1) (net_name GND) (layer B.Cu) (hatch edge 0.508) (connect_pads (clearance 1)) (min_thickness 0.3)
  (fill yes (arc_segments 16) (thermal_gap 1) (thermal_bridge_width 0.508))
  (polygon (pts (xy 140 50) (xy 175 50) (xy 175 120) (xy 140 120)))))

